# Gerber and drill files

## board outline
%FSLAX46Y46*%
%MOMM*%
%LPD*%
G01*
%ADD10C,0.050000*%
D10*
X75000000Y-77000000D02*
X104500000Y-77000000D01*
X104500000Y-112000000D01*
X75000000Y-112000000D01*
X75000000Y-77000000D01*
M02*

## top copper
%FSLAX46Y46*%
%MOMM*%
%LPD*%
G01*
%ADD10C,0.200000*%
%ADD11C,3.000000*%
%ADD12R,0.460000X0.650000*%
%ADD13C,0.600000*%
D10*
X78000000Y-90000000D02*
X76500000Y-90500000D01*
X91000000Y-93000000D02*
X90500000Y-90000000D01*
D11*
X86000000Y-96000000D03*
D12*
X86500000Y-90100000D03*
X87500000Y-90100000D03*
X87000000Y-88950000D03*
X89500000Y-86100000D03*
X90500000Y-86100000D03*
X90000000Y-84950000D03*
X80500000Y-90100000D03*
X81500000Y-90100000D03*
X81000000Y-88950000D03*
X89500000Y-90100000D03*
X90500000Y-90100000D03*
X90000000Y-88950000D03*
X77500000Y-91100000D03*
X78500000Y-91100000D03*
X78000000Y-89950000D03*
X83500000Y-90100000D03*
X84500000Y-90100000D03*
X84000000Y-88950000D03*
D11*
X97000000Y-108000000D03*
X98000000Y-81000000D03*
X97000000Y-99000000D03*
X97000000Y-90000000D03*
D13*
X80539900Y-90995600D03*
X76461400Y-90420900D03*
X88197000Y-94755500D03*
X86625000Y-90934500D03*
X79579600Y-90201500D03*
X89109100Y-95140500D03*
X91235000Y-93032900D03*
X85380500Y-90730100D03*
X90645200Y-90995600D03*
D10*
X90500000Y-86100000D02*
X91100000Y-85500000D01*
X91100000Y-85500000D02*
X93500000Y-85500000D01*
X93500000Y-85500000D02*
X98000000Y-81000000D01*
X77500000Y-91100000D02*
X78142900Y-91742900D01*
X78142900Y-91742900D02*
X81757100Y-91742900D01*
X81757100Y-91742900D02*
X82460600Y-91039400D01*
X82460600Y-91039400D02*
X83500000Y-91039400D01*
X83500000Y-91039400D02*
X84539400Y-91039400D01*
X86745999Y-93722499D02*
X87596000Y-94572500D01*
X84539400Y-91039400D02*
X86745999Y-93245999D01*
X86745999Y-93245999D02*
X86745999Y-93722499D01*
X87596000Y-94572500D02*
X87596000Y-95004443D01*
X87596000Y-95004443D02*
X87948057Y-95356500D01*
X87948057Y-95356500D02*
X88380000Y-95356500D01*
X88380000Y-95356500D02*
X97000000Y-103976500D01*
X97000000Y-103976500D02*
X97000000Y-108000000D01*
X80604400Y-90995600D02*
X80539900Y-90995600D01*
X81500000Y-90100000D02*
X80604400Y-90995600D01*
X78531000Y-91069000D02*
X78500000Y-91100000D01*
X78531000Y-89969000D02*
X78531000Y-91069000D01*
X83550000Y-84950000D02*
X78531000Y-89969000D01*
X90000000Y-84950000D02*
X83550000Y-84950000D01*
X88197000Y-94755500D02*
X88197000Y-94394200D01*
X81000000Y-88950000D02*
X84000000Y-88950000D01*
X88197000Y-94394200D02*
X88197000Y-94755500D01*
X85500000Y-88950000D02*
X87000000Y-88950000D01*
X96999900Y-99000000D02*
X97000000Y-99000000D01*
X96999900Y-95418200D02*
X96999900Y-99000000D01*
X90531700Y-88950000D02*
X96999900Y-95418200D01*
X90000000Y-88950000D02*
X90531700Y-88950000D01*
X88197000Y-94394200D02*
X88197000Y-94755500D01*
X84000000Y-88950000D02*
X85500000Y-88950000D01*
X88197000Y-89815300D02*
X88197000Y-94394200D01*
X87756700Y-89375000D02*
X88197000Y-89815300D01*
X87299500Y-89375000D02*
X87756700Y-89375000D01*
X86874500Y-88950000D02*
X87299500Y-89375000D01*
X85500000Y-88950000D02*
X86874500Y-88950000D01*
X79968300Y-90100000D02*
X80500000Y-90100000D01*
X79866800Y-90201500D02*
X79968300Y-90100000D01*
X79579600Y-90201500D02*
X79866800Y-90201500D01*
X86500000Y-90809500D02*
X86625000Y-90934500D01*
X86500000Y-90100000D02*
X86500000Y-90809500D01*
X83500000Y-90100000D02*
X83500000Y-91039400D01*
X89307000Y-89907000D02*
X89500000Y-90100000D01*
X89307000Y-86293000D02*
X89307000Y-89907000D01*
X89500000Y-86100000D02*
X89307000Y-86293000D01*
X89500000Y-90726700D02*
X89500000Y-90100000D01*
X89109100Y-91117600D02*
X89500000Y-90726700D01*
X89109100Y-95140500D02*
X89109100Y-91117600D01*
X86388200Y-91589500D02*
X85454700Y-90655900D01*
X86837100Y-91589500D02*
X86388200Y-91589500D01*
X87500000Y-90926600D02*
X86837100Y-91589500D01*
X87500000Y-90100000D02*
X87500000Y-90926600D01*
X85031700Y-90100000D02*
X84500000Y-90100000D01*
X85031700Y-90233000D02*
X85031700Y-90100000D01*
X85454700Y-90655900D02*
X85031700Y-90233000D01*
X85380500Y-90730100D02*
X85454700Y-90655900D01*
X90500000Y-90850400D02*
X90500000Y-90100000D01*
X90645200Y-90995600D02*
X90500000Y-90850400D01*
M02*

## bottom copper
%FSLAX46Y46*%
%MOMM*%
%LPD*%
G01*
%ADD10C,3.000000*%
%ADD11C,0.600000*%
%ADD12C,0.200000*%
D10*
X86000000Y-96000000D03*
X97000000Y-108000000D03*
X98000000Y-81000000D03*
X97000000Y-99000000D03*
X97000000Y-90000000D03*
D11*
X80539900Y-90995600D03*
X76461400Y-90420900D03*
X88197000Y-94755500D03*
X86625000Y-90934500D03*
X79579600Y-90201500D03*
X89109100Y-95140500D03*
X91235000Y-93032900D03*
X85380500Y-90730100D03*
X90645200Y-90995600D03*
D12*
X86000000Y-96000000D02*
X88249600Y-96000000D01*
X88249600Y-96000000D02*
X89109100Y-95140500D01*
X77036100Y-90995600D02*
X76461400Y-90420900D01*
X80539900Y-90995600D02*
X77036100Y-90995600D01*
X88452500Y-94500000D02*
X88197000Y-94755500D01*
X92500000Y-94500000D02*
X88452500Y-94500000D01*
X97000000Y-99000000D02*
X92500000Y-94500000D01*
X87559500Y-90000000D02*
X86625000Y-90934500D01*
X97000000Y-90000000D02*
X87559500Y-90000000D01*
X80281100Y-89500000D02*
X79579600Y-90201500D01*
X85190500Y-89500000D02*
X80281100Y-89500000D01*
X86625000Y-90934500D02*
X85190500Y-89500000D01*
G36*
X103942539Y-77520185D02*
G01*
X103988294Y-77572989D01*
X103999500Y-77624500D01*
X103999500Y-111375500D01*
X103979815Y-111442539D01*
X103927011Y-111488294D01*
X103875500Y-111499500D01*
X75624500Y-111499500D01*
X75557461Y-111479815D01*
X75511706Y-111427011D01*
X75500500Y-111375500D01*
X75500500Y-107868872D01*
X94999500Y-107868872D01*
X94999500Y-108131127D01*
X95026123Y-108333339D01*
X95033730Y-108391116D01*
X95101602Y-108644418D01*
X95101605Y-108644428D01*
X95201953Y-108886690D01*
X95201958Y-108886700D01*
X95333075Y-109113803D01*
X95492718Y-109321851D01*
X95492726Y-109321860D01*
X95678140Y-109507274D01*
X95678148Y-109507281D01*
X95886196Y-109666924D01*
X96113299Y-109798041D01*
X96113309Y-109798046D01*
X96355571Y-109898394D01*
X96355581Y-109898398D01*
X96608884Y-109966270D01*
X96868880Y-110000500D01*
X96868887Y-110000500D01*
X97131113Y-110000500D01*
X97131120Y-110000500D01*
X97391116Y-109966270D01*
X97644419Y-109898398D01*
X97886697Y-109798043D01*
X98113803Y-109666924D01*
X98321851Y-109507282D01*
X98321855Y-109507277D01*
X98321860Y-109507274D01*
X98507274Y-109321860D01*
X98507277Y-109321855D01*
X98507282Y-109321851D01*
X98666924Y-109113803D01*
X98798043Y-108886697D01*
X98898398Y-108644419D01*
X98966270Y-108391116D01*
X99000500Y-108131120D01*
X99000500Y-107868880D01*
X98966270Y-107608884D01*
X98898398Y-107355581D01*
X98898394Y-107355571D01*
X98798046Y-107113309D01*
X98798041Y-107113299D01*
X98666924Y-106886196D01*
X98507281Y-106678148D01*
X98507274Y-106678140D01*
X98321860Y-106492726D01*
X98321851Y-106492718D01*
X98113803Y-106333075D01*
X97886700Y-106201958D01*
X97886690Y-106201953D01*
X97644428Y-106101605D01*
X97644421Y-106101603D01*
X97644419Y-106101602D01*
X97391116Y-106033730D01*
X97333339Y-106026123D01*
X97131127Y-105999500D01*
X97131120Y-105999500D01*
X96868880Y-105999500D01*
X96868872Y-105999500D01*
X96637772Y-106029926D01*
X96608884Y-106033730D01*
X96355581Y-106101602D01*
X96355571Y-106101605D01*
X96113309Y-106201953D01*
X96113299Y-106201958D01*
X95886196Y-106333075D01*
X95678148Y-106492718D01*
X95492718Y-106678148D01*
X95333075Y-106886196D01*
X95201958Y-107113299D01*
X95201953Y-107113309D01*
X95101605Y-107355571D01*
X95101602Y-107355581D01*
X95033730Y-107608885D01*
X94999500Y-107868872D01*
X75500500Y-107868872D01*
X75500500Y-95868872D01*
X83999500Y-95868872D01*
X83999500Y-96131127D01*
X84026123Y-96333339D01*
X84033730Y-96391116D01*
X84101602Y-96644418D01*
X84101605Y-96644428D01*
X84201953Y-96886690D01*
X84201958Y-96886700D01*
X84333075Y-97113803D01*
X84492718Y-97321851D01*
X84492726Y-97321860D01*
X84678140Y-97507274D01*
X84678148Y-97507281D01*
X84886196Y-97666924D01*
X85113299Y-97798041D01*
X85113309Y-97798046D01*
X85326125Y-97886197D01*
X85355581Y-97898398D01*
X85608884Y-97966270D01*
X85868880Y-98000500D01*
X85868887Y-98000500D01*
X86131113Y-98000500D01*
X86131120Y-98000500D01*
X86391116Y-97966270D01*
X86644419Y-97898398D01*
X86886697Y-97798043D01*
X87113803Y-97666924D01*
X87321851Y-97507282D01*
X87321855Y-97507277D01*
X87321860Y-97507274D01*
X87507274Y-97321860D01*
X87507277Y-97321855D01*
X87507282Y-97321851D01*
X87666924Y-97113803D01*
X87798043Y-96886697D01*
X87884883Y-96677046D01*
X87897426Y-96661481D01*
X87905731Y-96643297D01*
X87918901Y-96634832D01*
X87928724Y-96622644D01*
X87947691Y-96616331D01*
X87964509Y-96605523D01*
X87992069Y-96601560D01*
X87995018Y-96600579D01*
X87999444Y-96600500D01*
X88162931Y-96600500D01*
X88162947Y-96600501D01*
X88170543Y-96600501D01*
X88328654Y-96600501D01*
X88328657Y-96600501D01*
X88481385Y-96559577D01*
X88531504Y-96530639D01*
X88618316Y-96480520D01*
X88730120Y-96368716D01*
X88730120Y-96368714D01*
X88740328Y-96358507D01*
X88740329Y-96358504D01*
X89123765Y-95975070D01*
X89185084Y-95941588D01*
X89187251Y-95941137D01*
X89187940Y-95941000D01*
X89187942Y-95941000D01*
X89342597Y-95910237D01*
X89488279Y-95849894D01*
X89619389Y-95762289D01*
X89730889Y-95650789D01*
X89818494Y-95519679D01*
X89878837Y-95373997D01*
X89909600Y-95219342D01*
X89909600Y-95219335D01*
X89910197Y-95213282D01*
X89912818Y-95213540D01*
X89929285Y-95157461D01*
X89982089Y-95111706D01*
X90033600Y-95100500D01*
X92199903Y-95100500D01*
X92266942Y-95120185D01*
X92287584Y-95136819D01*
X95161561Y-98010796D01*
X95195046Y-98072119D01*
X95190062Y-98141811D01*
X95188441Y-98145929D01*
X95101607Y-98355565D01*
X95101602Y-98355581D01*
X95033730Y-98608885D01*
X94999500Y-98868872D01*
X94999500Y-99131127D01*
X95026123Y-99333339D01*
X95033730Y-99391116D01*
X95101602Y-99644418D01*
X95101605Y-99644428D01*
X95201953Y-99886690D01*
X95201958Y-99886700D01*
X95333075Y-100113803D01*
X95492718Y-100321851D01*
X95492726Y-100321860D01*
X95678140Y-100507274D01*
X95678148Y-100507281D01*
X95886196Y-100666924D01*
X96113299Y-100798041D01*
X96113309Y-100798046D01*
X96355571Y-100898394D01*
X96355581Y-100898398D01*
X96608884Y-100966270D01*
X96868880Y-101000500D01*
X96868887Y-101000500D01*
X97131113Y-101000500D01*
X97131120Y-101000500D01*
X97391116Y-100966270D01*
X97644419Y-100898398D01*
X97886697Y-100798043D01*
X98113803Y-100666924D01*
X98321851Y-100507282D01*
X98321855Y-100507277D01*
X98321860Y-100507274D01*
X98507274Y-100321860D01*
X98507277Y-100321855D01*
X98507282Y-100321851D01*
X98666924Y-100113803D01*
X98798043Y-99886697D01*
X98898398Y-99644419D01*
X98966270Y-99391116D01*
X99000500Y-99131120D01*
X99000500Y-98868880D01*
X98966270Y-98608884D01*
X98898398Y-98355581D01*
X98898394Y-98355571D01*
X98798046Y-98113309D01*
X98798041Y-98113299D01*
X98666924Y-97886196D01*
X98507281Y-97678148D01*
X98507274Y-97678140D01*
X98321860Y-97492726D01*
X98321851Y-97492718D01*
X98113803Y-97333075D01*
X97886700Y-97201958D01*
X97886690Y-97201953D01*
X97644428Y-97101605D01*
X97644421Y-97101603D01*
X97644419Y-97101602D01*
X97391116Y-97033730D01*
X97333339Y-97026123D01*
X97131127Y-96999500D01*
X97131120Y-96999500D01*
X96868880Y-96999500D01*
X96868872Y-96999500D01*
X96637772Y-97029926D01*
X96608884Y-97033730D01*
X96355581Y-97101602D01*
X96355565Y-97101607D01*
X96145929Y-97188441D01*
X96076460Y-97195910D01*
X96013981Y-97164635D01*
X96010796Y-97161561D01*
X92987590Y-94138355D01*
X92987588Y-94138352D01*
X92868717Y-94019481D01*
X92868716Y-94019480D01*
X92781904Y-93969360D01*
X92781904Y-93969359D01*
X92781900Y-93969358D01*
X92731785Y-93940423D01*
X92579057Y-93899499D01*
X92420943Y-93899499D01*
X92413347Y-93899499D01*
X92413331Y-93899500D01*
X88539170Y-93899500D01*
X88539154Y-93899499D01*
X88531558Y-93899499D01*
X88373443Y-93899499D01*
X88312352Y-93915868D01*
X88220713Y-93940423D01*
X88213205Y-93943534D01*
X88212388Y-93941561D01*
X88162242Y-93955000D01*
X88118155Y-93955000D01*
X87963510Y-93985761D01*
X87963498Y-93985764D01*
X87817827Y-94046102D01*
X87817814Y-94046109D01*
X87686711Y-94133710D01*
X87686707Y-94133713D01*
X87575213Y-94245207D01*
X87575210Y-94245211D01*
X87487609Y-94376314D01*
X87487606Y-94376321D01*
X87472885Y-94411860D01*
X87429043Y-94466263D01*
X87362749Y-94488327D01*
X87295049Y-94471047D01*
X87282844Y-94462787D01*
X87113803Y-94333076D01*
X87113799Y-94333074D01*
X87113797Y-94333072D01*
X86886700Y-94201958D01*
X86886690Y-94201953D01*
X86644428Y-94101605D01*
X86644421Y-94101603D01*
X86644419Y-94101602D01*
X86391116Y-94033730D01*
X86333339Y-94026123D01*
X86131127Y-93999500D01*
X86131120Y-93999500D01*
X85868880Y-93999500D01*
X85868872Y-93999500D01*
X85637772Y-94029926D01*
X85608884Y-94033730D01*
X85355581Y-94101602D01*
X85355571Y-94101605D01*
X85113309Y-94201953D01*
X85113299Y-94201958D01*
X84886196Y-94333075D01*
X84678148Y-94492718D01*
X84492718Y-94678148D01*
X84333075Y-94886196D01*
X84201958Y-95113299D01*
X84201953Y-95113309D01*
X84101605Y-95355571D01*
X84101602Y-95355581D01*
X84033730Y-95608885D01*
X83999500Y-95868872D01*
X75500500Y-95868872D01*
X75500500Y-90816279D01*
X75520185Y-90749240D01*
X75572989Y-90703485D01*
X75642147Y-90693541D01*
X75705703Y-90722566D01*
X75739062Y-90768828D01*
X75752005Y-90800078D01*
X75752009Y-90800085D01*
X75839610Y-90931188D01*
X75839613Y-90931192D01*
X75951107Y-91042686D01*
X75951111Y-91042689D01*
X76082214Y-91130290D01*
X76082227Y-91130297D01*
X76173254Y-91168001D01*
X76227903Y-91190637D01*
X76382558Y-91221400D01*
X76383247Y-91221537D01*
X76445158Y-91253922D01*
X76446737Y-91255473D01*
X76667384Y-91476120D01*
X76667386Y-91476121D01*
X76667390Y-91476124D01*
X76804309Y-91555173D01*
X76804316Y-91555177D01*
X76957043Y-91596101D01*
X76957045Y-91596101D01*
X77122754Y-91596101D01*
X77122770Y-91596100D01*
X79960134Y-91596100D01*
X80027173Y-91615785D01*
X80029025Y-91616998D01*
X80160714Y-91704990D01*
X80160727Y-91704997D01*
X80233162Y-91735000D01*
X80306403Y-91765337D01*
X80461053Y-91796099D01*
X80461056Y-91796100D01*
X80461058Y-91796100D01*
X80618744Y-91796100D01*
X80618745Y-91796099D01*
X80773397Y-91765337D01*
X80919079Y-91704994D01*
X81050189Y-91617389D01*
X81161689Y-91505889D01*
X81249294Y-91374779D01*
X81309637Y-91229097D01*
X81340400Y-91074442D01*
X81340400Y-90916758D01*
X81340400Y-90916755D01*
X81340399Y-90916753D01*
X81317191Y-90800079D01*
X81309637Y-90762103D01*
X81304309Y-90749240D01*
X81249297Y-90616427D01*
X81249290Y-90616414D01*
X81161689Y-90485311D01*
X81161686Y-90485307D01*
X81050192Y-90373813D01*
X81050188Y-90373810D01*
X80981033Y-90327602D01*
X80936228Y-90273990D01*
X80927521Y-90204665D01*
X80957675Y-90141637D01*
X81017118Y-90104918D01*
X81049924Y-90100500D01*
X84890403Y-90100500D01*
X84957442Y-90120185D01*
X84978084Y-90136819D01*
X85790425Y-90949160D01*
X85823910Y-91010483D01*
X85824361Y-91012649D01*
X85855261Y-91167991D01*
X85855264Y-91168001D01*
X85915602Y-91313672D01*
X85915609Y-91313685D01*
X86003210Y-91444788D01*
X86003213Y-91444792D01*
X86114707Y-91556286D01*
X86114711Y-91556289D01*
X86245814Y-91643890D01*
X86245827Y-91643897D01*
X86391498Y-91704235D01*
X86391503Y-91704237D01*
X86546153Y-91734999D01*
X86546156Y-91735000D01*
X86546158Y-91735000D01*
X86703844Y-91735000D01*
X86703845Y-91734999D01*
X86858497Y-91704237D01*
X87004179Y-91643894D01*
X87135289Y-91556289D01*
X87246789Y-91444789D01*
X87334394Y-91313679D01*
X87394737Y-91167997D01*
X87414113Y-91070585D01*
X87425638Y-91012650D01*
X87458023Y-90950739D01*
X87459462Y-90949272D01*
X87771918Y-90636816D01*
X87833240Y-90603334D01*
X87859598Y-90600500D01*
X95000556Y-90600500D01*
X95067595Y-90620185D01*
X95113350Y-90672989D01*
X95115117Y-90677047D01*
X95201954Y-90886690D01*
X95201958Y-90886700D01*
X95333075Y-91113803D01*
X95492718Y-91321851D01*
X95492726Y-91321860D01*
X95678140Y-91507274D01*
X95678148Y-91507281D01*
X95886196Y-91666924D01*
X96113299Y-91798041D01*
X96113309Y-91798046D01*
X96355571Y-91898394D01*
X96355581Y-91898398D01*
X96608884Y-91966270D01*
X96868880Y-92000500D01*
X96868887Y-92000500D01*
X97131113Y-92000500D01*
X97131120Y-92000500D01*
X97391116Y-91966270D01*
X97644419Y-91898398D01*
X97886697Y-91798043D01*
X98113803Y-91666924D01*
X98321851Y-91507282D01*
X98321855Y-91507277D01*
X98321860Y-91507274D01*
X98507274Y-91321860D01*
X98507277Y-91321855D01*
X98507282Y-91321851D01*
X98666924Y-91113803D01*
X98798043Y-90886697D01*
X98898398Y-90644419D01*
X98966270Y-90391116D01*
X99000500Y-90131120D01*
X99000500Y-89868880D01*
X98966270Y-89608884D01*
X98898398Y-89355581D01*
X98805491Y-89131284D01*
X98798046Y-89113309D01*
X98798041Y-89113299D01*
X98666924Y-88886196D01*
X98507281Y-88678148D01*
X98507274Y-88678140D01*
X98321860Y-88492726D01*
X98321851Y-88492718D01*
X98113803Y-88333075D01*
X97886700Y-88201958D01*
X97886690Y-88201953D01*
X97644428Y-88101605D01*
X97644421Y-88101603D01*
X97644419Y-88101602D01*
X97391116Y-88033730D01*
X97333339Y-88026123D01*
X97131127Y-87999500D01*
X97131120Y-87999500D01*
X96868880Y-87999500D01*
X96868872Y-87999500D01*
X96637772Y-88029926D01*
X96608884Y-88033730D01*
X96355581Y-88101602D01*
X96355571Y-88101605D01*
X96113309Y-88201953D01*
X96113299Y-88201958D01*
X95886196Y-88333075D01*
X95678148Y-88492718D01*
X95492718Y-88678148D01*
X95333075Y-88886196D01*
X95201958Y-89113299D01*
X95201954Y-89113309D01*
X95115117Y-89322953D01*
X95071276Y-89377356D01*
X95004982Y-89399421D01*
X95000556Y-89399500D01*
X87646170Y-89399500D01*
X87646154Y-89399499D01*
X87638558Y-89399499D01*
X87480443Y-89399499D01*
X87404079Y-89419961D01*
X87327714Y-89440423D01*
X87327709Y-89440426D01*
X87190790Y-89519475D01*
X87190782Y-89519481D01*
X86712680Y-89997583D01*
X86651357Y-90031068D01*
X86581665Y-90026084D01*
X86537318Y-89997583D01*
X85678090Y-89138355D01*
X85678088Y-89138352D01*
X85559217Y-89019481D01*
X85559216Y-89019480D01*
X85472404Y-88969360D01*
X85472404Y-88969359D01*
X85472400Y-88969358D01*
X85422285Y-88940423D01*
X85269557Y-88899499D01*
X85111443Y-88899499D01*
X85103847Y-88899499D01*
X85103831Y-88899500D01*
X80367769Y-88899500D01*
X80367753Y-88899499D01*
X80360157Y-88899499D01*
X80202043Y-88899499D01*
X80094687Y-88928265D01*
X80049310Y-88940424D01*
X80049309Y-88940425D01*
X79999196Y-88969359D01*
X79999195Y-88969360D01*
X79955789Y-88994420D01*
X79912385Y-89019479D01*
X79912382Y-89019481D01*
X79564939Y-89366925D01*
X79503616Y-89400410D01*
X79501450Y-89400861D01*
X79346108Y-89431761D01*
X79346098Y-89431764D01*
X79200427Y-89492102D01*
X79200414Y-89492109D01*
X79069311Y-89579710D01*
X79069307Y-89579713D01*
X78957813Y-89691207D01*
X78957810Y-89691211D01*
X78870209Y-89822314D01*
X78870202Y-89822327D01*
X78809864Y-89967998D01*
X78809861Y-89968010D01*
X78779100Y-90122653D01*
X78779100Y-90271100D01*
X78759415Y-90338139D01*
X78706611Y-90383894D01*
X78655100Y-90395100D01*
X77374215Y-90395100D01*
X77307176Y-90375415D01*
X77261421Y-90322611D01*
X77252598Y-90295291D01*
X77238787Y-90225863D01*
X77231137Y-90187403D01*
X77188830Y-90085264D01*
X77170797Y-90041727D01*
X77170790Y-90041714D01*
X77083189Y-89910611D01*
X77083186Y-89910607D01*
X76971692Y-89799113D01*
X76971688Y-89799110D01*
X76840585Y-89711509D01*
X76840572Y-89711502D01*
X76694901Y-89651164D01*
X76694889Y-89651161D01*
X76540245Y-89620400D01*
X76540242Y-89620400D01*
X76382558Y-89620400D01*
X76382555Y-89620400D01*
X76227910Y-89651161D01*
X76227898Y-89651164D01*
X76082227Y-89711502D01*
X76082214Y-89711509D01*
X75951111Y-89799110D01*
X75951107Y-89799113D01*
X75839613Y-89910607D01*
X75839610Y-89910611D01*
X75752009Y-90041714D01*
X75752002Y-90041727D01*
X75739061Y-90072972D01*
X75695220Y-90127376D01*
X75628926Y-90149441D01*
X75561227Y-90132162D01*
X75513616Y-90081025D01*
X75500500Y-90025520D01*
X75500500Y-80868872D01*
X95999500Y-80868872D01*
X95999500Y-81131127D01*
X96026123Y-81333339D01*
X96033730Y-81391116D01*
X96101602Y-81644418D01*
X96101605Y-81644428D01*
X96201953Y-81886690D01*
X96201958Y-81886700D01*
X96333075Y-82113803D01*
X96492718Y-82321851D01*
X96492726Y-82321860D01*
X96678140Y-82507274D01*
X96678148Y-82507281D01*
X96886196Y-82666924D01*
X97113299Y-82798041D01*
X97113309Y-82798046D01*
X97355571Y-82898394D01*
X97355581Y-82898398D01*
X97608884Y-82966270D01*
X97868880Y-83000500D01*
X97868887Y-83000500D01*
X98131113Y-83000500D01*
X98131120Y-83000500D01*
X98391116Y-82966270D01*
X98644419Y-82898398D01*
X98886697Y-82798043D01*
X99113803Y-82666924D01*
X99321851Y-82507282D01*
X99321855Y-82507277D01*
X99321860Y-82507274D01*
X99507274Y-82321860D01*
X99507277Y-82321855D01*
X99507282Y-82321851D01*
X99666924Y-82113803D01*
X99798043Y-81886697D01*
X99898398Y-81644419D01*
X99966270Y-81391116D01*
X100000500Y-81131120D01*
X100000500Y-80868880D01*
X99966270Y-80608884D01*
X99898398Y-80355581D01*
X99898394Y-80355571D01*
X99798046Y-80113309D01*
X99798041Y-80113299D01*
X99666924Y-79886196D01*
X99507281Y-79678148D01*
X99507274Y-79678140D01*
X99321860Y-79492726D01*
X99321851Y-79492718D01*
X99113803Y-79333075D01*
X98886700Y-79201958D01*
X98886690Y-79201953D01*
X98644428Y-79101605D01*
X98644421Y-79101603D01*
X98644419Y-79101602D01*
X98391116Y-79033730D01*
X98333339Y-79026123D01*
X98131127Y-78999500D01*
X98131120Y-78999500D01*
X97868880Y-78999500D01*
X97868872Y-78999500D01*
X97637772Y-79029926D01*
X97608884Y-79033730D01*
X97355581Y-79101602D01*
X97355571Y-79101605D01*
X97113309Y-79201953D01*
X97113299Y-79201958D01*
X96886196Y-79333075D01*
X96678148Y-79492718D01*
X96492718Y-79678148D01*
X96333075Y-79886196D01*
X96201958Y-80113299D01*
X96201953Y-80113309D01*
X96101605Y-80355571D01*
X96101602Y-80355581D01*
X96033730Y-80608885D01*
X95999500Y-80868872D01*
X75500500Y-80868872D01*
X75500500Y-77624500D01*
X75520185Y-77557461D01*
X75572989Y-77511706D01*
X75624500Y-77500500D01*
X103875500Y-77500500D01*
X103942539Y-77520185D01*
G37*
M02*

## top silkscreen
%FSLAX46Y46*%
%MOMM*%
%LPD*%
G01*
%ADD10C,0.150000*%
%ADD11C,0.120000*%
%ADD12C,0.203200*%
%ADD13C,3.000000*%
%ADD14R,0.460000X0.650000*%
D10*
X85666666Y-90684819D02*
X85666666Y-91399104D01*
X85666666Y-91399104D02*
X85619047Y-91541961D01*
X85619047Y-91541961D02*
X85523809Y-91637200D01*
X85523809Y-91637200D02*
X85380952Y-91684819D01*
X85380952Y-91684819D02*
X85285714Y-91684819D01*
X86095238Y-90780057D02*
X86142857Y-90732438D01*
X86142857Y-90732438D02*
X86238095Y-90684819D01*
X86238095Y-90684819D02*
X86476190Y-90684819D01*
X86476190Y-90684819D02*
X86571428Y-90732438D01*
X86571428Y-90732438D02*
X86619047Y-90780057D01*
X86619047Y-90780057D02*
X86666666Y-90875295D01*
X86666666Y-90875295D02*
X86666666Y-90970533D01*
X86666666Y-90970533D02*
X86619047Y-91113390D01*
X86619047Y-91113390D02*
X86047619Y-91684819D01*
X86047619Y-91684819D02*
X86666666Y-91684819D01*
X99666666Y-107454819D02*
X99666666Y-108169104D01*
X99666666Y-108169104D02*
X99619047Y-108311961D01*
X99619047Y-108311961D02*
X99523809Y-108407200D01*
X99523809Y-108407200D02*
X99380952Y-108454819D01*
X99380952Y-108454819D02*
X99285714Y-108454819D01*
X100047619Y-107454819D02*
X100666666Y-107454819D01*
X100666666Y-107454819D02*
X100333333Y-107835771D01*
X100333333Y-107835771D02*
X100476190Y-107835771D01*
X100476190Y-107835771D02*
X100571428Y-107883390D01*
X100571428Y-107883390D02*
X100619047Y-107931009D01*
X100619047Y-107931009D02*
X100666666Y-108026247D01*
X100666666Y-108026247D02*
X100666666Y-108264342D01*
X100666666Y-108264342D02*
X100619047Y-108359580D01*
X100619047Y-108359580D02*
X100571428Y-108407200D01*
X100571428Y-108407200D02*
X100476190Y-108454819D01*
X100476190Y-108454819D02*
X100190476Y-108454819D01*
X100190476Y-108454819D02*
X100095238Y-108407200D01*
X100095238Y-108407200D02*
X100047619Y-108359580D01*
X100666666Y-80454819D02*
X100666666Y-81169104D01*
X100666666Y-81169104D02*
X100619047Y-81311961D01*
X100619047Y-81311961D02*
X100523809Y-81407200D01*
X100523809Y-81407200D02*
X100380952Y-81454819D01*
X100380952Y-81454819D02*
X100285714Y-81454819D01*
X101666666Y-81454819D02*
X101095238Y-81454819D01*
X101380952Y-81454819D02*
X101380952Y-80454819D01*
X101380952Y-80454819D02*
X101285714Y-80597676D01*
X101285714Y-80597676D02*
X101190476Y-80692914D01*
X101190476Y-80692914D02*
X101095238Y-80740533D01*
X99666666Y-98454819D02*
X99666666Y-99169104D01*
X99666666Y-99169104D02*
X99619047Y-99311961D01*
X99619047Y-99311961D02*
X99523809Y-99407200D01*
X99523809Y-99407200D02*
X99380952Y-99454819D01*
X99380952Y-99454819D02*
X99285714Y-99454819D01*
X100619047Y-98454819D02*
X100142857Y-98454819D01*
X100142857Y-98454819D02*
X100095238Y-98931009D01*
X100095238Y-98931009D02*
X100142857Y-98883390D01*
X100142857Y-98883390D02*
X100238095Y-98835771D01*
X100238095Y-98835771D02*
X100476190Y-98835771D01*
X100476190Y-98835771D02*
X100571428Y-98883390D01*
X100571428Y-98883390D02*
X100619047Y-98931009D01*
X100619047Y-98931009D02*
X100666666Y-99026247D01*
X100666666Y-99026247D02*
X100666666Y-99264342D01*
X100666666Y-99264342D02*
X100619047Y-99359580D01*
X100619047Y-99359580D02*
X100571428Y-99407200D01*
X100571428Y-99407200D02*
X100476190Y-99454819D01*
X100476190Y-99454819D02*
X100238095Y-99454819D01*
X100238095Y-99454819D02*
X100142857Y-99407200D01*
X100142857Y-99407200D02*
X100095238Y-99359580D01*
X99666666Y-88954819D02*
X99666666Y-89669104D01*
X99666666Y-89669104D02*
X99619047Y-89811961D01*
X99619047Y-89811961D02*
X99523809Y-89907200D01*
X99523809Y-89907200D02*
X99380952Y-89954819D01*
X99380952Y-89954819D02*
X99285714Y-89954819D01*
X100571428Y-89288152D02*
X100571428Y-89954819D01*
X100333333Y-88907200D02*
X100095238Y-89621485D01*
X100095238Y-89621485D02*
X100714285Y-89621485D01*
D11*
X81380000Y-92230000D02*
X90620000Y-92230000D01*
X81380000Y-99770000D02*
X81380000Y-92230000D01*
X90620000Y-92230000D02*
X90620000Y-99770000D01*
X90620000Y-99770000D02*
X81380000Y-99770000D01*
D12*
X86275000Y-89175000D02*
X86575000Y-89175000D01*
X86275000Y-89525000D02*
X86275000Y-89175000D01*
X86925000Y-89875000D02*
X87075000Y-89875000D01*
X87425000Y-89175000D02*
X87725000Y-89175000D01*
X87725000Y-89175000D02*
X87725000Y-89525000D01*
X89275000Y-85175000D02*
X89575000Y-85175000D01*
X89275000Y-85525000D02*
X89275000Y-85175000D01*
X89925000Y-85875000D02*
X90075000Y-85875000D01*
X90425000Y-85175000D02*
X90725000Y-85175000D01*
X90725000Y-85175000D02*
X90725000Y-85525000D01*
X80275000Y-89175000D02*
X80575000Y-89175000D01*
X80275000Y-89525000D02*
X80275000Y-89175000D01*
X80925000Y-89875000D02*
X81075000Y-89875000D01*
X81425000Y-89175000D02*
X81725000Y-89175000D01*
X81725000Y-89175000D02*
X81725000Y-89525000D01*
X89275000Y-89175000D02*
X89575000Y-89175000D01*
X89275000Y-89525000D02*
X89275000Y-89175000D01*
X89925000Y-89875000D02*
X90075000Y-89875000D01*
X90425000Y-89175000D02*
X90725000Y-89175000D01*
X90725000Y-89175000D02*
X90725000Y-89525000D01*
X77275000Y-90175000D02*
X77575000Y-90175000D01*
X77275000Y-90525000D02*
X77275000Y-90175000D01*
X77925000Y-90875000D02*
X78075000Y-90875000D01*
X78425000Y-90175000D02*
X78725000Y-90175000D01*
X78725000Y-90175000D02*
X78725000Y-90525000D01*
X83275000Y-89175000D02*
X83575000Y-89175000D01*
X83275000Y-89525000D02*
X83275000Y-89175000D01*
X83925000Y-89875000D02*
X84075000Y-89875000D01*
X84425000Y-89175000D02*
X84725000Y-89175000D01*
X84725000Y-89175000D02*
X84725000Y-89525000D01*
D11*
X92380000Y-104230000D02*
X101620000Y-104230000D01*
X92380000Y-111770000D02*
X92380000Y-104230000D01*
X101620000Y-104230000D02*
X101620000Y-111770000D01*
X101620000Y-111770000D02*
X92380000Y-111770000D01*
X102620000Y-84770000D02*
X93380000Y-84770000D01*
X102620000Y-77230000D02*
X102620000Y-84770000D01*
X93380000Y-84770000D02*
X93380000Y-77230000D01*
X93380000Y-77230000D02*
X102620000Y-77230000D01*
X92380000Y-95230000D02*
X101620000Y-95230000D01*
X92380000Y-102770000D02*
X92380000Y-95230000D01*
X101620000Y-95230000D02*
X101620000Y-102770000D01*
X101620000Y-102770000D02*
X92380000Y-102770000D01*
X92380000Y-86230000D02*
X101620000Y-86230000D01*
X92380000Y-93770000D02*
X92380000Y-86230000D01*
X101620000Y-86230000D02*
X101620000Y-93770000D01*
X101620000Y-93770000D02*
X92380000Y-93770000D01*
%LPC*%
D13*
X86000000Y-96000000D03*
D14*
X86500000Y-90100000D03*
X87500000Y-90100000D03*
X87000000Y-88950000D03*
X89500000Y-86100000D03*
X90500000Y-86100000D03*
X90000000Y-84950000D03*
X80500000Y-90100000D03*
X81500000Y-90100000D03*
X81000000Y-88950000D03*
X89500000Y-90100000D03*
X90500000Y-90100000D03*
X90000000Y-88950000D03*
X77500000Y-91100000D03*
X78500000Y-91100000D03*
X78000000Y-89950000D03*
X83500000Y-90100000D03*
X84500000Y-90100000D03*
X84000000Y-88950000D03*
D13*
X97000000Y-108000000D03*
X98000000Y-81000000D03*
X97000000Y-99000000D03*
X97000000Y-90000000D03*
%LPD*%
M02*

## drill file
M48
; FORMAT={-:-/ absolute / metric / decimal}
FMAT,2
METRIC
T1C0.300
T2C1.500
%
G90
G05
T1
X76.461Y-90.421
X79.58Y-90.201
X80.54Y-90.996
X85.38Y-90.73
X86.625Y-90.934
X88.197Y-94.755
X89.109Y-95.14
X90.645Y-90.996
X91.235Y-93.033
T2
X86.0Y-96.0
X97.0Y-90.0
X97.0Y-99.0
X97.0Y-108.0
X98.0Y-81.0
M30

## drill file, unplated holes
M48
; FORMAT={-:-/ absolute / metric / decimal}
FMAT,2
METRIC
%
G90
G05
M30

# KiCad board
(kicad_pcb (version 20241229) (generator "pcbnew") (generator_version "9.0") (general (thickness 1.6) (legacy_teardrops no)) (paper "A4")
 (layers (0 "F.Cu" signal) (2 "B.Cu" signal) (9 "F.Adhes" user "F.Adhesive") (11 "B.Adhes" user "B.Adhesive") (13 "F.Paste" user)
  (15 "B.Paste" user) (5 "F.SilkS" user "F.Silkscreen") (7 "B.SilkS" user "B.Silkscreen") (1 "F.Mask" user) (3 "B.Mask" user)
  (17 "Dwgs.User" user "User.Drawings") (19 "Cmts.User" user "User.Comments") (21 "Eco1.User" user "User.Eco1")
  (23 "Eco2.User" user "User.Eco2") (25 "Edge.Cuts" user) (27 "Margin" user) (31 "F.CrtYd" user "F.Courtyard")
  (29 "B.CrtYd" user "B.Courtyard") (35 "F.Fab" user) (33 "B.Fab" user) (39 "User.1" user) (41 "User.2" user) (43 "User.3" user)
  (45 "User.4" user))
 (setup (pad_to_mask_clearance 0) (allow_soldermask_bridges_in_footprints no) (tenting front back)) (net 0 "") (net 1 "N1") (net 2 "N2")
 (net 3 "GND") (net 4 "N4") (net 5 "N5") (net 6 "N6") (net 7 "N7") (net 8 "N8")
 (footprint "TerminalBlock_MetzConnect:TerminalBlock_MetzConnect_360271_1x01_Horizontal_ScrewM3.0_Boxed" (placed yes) (layer "F.Cu")
  (at 86 96)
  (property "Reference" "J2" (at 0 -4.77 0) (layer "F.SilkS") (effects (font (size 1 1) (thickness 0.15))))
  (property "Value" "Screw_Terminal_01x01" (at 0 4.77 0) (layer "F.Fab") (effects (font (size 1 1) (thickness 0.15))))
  (fp_line (start -4.62 -3.77) (end 4.62 -3.77) (stroke (width 0.12) (type solid)) (layer "F.SilkS"))
  (fp_line (start -4.62 3.77) (end -4.62 -3.77) (stroke (width 0.12) (type solid)) (layer "F.SilkS"))
  (fp_line (start 4.62 -3.77) (end 4.62 3.77) (stroke (width 0.12) (type solid)) (layer "F.SilkS"))
  (fp_line (start 4.62 3.77) (end -4.62 3.77) (stroke (width 0.12) (type solid)) (layer "F.SilkS"))
  (pad "1" thru_hole circle (at 0 0) (size 3 3) (drill 1.5) (layers "*.Cu" "*.Mask") (remove_unused_layers no) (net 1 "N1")))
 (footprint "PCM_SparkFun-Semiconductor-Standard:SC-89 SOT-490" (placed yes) (layer "F.Cu") (at 87 89)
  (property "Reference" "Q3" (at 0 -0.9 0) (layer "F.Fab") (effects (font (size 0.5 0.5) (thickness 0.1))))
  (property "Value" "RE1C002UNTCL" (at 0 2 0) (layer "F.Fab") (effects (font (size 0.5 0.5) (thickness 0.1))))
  (fp_line (start -0.725 0.175) (end -0.425 0.175) (stroke (width 0.2032) (type solid)) (layer "F.SilkS"))
  (fp_line (start -0.725 0.525) (end -0.725 0.175) (stroke (width 0.2032) (type solid)) (layer "F.SilkS"))
  (fp_line (start -0.075 0.875) (end 0.075 0.875) (stroke (width 0.2032) (type solid)) (layer "F.SilkS"))
  (fp_line (start 0.425 0.175) (end 0.725 0.175) (stroke (width 0.2032) (type solid)) (layer "F.SilkS"))
  (fp_line (start 0.725 0.175) (end 0.725 0.525) (stroke (width 0.2032) (type solid)) (layer "F.SilkS"))
  (pad "1" smd rect (at -0.5 1.1) (size 0.46 0.65) (layers "F.Cu" "F.Mask" "F.Paste") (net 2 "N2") (thermal_bridge_angle 0))
  (pad "2" smd rect (at 0.5 1.1) (size 0.46 0.65) (layers "F.Cu" "F.Mask" "F.Paste") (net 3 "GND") (thermal_bridge_angle 0))
  (pad "3" smd rect (at 0 -0.05) (size 0.46 0.65) (layers "F.Cu" "F.Mask" "F.Paste") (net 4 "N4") (thermal_bridge_angle 0)))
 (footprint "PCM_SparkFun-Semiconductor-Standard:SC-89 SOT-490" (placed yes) (layer "F.Cu") (at 90 85)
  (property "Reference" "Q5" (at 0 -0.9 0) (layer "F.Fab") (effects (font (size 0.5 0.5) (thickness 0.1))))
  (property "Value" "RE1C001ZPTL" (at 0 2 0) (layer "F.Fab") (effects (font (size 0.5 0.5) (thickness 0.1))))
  (fp_line (start -0.725 0.175) (end -0.425 0.175) (stroke (width 0.2032) (type solid)) (layer "F.SilkS"))
  (fp_line (start -0.725 0.525) (end -0.725 0.175) (stroke (width 0.2032) (type solid)) (layer "F.SilkS"))
  (fp_line (start -0.075 0.875) (end 0.075 0.875) (stroke (width 0.2032) (type solid)) (layer "F.SilkS"))
  (fp_line (start 0.425 0.175) (end 0.725 0.175) (stroke (width 0.2032) (type solid)) (layer "F.SilkS"))
  (fp_line (start 0.725 0.175) (end 0.725 0.525) (stroke (width 0.2032) (type solid)) (layer "F.SilkS"))
  (pad "1" smd rect (at -0.5 1.1) (size 0.46 0.65) (layers "F.Cu" "F.Mask" "F.Paste") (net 1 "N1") (thermal_bridge_angle 0))
  (pad "2" smd rect (at 0.5 1.1) (size 0.46 0.65) (layers "F.Cu" "F.Mask" "F.Paste") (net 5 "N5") (thermal_bridge_angle 0))
  (pad "3" smd rect (at 0 -0.05) (size 0.46 0.65) (layers "F.Cu" "F.Mask" "F.Paste") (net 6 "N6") (thermal_bridge_angle 0)))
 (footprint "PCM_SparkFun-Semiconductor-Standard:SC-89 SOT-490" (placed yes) (layer "F.Cu") (at 81 89)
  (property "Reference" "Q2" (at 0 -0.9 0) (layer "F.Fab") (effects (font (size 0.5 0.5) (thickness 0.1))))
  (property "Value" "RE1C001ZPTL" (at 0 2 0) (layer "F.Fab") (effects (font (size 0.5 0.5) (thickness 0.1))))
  (fp_line (start -0.725 0.175) (end -0.425 0.175) (stroke (width 0.2032) (type solid)) (layer "F.SilkS"))
  (fp_line (start -0.725 0.525) (end -0.725 0.175) (stroke (width 0.2032) (type solid)) (layer "F.SilkS"))
  (fp_line (start -0.075 0.875) (end 0.075 0.875) (stroke (width 0.2032) (type solid)) (layer "F.SilkS"))
  (fp_line (start 0.425 0.175) (end 0.725 0.175) (stroke (width 0.2032) (type solid)) (layer "F.SilkS"))
  (fp_line (start 0.725 0.175) (end 0.725 0.525) (stroke (width 0.2032) (type solid)) (layer "F.SilkS"))
  (pad "1" smd rect (at -0.5 1.1) (size 0.46 0.65) (layers "F.Cu" "F.Mask" "F.Paste") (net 2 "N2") (thermal_bridge_angle 0))
  (pad "2" smd rect (at 0.5 1.1) (size 0.46 0.65) (layers "F.Cu" "F.Mask" "F.Paste") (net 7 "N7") (thermal_bridge_angle 0))
  (pad "3" smd rect (at 0 -0.05) (size 0.46 0.65) (layers "F.Cu" "F.Mask" "F.Paste") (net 4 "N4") (thermal_bridge_angle 0)))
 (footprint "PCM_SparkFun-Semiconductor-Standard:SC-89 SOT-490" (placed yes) (layer "F.Cu") (at 90 89)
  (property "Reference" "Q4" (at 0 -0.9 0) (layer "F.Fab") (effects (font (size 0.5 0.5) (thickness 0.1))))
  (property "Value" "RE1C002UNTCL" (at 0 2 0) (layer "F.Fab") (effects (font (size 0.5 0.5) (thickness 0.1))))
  (fp_line (start -0.725 0.175) (end -0.425 0.175) (stroke (width 0.2032) (type solid)) (layer "F.SilkS"))
  (fp_line (start -0.725 0.525) (end -0.725 0.175) (stroke (width 0.2032) (type solid)) (layer "F.SilkS"))
  (fp_line (start -0.075 0.875) (end 0.075 0.875) (stroke (width 0.2032) (type solid)) (layer "F.SilkS"))
  (fp_line (start 0.425 0.175) (end 0.725 0.175) (stroke (width 0.2032) (type solid)) (layer "F.SilkS"))
  (fp_line (start 0.725 0.175) (end 0.725 0.525) (stroke (width 0.2032) (type solid)) (layer "F.SilkS"))
  (pad "1" smd rect (at -0.5 1.1) (size 0.46 0.65) (layers "F.Cu" "F.Mask" "F.Paste") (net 1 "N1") (thermal_bridge_angle 0))
  (pad "2" smd rect (at 0.5 1.1) (size 0.46 0.65) (layers "F.Cu" "F.Mask" "F.Paste") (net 3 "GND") (thermal_bridge_angle 0))
  (pad "3" smd rect (at 0 -0.05) (size 0.46 0.65) (layers "F.Cu" "F.Mask" "F.Paste") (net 4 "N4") (thermal_bridge_angle 0)))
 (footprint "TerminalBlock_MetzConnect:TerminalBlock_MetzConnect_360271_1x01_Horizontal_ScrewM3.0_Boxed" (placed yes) (layer "F.Cu")
  (at 97 90)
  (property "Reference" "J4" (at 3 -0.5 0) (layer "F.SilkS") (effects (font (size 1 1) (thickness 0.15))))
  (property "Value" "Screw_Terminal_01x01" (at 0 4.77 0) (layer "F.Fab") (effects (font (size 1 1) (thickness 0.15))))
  (fp_line (start -4.62 -3.77) (end 4.62 -3.77) (stroke (width 0.12) (type solid)) (layer "F.SilkS"))
  (fp_line (start -4.62 3.77) (end -4.62 -3.77) (stroke (width 0.12) (type solid)) (layer "F.SilkS"))
  (fp_line (start 4.62 -3.77) (end 4.62 3.77) (stroke (width 0.12) (type solid)) (layer "F.SilkS"))
  (fp_line (start 4.62 3.77) (end -4.62 3.77) (stroke (width 0.12) (type solid)) (layer "F.SilkS"))
  (pad "1" thru_hole circle (at 0 0) (size 3 3) (drill 1.5) (layers "*.Cu" "*.Mask") (remove_unused_layers no) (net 2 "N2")))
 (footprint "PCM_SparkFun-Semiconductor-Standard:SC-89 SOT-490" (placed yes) (layer "F.Cu") (at 78 90)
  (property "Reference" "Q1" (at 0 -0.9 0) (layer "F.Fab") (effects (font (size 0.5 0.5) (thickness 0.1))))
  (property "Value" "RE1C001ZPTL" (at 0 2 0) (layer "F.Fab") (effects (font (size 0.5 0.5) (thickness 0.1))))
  (fp_line (start -0.725 0.175) (end -0.425 0.175) (stroke (width 0.2032) (type solid)) (layer "F.SilkS"))
  (fp_line (start -0.725 0.525) (end -0.725 0.175) (stroke (width 0.2032) (type solid)) (layer "F.SilkS"))
  (fp_line (start -0.075 0.875) (end 0.075 0.875) (stroke (width 0.2032) (type solid)) (layer "F.SilkS"))
  (fp_line (start 0.425 0.175) (end 0.725 0.175) (stroke (width 0.2032) (type solid)) (layer "F.SilkS"))
  (fp_line (start 0.725 0.175) (end 0.725 0.525) (stroke (width 0.2032) (type solid)) (layer "F.SilkS"))
  (pad "1" smd rect (at -0.5 1.1) (size 0.46 0.65) (layers "F.Cu" "F.Mask" "F.Paste") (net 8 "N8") (thermal_bridge_angle 0))
  (pad "2" smd rect (at 0.5 1.1) (size 0.46 0.65) (layers "F.Cu" "F.Mask" "F.Paste") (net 6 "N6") (thermal_bridge_angle 0))
  (pad "3" smd rect (at 0 -0.05) (size 0.46 0.65) (layers "F.Cu" "F.Mask" "F.Paste") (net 7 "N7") (thermal_bridge_angle 0)))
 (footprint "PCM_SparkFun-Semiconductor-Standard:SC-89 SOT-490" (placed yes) (layer "F.Cu") (at 84 89)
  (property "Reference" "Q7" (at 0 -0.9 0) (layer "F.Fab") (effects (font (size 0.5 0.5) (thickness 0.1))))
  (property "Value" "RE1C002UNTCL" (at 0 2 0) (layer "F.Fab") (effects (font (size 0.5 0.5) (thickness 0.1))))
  (fp_line (start -0.725 0.175) (end -0.425 0.175) (stroke (width 0.2032) (type solid)) (layer "F.SilkS"))
  (fp_line (start -0.725 0.525) (end -0.725 0.175) (stroke (width 0.2032) (type solid)) (layer "F.SilkS"))
  (fp_line (start -0.075 0.875) (end 0.075 0.875) (stroke (width 0.2032) (type solid)) (layer "F.SilkS"))
  (fp_line (start 0.425 0.175) (end 0.725 0.175) (stroke (width 0.2032) (type solid)) (layer "F.SilkS"))
  (fp_line (start 0.725 0.175) (end 0.725 0.525) (stroke (width 0.2032) (type solid)) (layer "F.SilkS"))
  (pad "1" smd rect (at -0.5 1.1) (size 0.46 0.65) (layers "F.Cu" "F.Mask" "F.Paste") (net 8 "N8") (thermal_bridge_angle 0))
  (pad "2" smd rect (at 0.5 1.1) (size 0.46 0.65) (layers "F.Cu" "F.Mask" "F.Paste") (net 3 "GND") (thermal_bridge_angle 0))
  (pad "3" smd rect (at 0 -0.05) (size 0.46 0.65) (layers "F.Cu" "F.Mask" "F.Paste") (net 4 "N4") (thermal_bridge_angle 0)))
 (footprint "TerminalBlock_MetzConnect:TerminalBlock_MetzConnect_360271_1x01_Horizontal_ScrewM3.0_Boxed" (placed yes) (layer "F.Cu")
  (at 97 108)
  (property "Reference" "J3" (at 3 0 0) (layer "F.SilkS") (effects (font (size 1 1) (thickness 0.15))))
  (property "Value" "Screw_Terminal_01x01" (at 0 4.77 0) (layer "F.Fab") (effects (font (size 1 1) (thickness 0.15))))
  (fp_line (start -4.62 -3.77) (end 4.62 -3.77) (stroke (width 0.12) (type solid)) (layer "F.SilkS"))
  (fp_line (start -4.62 3.77) (end -4.62 -3.77) (stroke (width 0.12) (type solid)) (layer "F.SilkS"))
  (fp_line (start 4.62 -3.77) (end 4.62 3.77) (stroke (width 0.12) (type solid)) (layer "F.SilkS"))
  (fp_line (start 4.62 3.77) (end -4.62 3.77) (stroke (width 0.12) (type solid)) (layer "F.SilkS"))
  (pad "1" thru_hole circle (at 0 0) (size 3 3) (drill 1.5) (layers "*.Cu" "*.Mask") (remove_unused_layers no) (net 8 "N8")))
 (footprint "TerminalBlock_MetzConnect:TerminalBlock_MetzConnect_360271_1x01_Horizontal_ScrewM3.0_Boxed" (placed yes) (layer "F.Cu")
  (at 98 81)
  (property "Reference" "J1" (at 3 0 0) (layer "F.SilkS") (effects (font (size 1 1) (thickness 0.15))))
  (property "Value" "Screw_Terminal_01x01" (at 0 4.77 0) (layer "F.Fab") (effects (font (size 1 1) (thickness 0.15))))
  (fp_line (start -4.62 -3.77) (end 4.62 -3.77) (stroke (width 0.12) (type solid)) (layer "F.SilkS"))
  (fp_line (start -4.62 3.77) (end -4.62 -3.77) (stroke (width 0.12) (type solid)) (layer "F.SilkS"))
  (fp_line (start 4.62 -3.77) (end 4.62 3.77) (stroke (width 0.12) (type solid)) (layer "F.SilkS"))
  (fp_line (start 4.62 3.77) (end -4.62 3.77) (stroke (width 0.12) (type solid)) (layer "F.SilkS"))
  (pad "1" thru_hole circle (at 0 0) (size 3 3) (drill 1.5) (layers "*.Cu" "*.Mask") (remove_unused_layers no) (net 5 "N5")))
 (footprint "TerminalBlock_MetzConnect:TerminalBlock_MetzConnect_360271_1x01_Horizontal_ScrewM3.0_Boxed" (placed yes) (layer "F.Cu")
  (at 97 99)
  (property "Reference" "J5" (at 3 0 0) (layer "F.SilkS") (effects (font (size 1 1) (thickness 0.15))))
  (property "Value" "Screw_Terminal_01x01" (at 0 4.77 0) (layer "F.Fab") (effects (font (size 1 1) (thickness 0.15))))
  (fp_line (start -4.62 -3.77) (end 4.62 -3.77) (stroke (width 0.12) (type solid)) (layer "F.SilkS"))
  (fp_line (start -4.62 3.77) (end -4.62 -3.77) (stroke (width 0.12) (type solid)) (layer "F.SilkS"))
  (fp_line (start 4.62 -3.77) (end 4.62 3.77) (stroke (width 0.12) (type solid)) (layer "F.SilkS"))
  (fp_line (start 4.62 3.77) (end -4.62 3.77) (stroke (width 0.12) (type solid)) (layer "F.SilkS"))
  (pad "1" thru_hole circle (at 0 0) (size 3 3) (drill 1.5) (layers "*.Cu" "*.Mask") (remove_unused_layers no) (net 4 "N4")))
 (gr_line (start 91 93) (end 90.5 90) (stroke (width 0.2) (type default)) (layer "F.Cu") (net 3))
 (gr_line (start 78 90) (end 76.5 90.5) (stroke (width 0.2) (type default)) (layer "F.Cu") (net 7))
 (gr_rect (start 75 77) (end 104.5 112) (stroke (width 0.05) (type default)) (fill no) (layer "Edge.Cuts"))
 (segment (start 90.5 86.1) (end 91.1 85.5) (width 0.2) (layer "F.Cu") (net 5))
 (segment (start 93.5 85.5) (end 98 81) (width 0.2) (layer "F.Cu") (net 5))
 (segment (start 91.1 85.5) (end 93.5 85.5) (width 0.2) (layer "F.Cu") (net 5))
 (segment (start 89.307 86.293) (end 89.307 89.907) (width 0.2) (layer "F.Cu") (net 1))
 (segment (start 89.5 86.1) (end 89.307 86.293) (width 0.2) (layer "F.Cu") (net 1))
 (segment (start 89.307 89.907) (end 89.5 90.1) (width 0.2) (layer "F.Cu") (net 1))
 (segment (start 89.1091 91.1176) (end 89.5 90.7267) (width 0.2) (layer "F.Cu") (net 1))
 (segment (start 89.1091 95.1405) (end 89.1091 91.1176) (width 0.2) (layer "F.Cu") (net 1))
 (segment (start 89.5 90.7267) (end 89.5 90.1) (width 0.2) (layer "F.Cu") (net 1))
 (via (at 89.1091 95.1405) (size 0.6) (drill 0.3) (layers "F.Cu" "B.Cu") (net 1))
 (segment (start 86 96) (end 88.2496 96) (width 0.2) (layer "B.Cu") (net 1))
 (segment (start 88.2496 96) (end 89.1091 95.1405) (width 0.2) (layer "B.Cu") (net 1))
 (segment (start 77.5 91.1) (end 78.1429 91.7429) (width 0.2) (layer "F.Cu") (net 8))
 (segment (start 83.5 91.0394) (end 84.5394 91.0394) (width 0.2) (layer "F.Cu") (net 8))
 (segment (start 88.38 95.3565) (end 97 103.9765) (width 0.2) (layer "F.Cu") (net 8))
 (segment (start 86.745999 93.245999) (end 86.745999 93.722499) (width 0.2) (layer "F.Cu") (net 8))
 (segment (start 87.948057 95.3565) (end 88.38 95.3565) (width 0.2) (layer "F.Cu") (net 8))
 (segment (start 83.5 90.1) (end 83.5 91.0394) (width 0.2) (layer "F.Cu") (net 8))
 (segment (start 87.596 94.5725) (end 87.596 95.004443) (width 0.2) (layer "F.Cu") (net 8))
 (segment (start 81.7571 91.7429) (end 82.4606 91.0394) (width 0.2) (layer "F.Cu") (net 8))
 (segment (start 84.5394 91.0394) (end 86.745999 93.245999) (width 0.2) (layer "F.Cu") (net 8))
 (segment (start 82.4606 91.0394) (end 83.5 91.0394) (width 0.2) (layer "F.Cu") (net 8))
 (segment (start 97 103.9765) (end 97 108) (width 0.2) (layer "F.Cu") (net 8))
 (segment (start 78.1429 91.7429) (end 81.7571 91.7429) (width 0.2) (layer "F.Cu") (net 8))
 (segment (start 86.745999 93.722499) (end 87.596 94.5725) (width 0.2) (layer "F.Cu") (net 8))
 (segment (start 87.596 95.004443) (end 87.948057 95.3565) (width 0.2) (layer "F.Cu") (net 8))
 (segment (start 79.5796 90.2015) (end 79.8668 90.2015) (width 0.2) (layer "F.Cu") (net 2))
 (segment (start 79.9683 90.1) (end 80.5 90.1) (width 0.2) (layer "F.Cu") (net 2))
 (segment (start 86.5 90.8095) (end 86.625 90.9345) (width 0.2) (layer "F.Cu") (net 2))
 (segment (start 79.8668 90.2015) (end 79.9683 90.1) (width 0.2) (layer "F.Cu") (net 2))
 (segment (start 86.5 90.1) (end 86.5 90.8095) (width 0.2) (layer "F.Cu") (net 2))
 (via (at 79.5796 90.2015) (size 0.6) (drill 0.3) (layers "F.Cu" "B.Cu") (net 2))
 (via (at 86.625 90.9345) (size 0.6) (drill 0.3) (layers "F.Cu" "B.Cu") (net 2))
 (segment (start 80.2811 89.5) (end 79.5796 90.2015) (width 0.2) (layer "B.Cu") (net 2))
 (segment (start 87.5595 90) (end 86.625 90.9345) (width 0.2) (layer "B.Cu") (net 2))
 (segment (start 97 90) (end 87.5595 90) (width 0.2) (layer "B.Cu") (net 2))
 (segment (start 86.625 90.9345) (end 85.1905 89.5) (width 0.2) (layer "B.Cu") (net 2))
 (segment (start 85.1905 89.5) (end 80.2811 89.5) (width 0.2) (layer "B.Cu") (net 2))
 (segment (start 90 88.95) (end 90.5317 88.95) (width 0.2) (layer "F.Cu") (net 4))
 (segment (start 96.9999 99) (end 97 99) (width 0.2) (layer "F.Cu") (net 4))
 (segment (start 84 88.95) (end 85.5 88.95) (width 0.2) (layer "F.Cu") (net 4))
 (segment (start 88.197 89.8153) (end 88.197 94.3942) (width 0.2) (layer "F.Cu") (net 4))
 (segment (start 90.5317 88.95) (end 96.9999 95.4182) (width 0.2) (layer "F.Cu") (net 4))
 (segment (start 86.8745 88.95) (end 87.2995 89.375) (width 0.2) (layer "F.Cu") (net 4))
 (segment (start 87.2995 89.375) (end 87.7567 89.375) (width 0.2) (layer "F.Cu") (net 4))
 (segment (start 81 88.95) (end 84 88.95) (width 0.2) (layer "F.Cu") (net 4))
 (segment (start 85.5 88.95) (end 87 88.95) (width 0.2) (layer "F.Cu") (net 4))
 (segment (start 88.197 94.3942) (end 88.197 94.7555) (width 0.2) (layer "F.Cu") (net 4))
 (segment (start 85.5 88.95) (end 86.8745 88.95) (width 0.2) (layer "F.Cu") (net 4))
 (segment (start 87.7567 89.375) (end 88.197 89.8153) (width 0.2) (layer "F.Cu") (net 4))
 (segment (start 88.197 94.3942) (end 88.197 94.7555) (width 0.2) (layer "F.Cu") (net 4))
 (segment (start 88.197 94.7555) (end 88.197 94.3942) (width 0.2) (layer "F.Cu") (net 4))
 (segment (start 96.9999 95.4182) (end 96.9999 99) (width 0.2) (layer "F.Cu") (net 4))
 (via (at 88.197 94.7555) (size 0.6) (drill 0.3) (layers "F.Cu" "B.Cu") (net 4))
 (segment (start 92.5 94.5) (end 88.4525 94.5) (width 0.2) (layer "B.Cu") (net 4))
 (segment (start 88.4525 94.5) (end 88.197 94.7555) (width 0.2) (layer "B.Cu") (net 4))
 (segment (start 97 99) (end 92.5 94.5) (width 0.2) (layer "B.Cu") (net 4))
 (segment (start 78.531 91.069) (end 78.5 91.1) (width 0.2) (layer "F.Cu") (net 6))
 (segment (start 83.55 84.95) (end 78.531 89.969) (width 0.2) (layer "F.Cu") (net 6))
 (segment (start 90 84.95) (end 83.55 84.95) (width 0.2) (layer "F.Cu") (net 6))
 (segment (start 78.531 89.969) (end 78.531 91.069) (width 0.2) (layer "F.Cu") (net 6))
 (segment (start 81.5 90.1) (end 80.6044 90.9956) (width 0.2) (layer "F.Cu") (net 7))
 (segment (start 80.6044 90.9956) (end 80.5399 90.9956) (width 0.2) (layer "F.Cu") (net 7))
 (via (at 76.4614 90.4209) (size 0.6) (drill 0.3) (layers "F.Cu" "B.Cu") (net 7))
 (via (at 80.5399 90.9956) (size 0.6) (drill 0.3) (layers "F.Cu" "B.Cu") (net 7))
 (segment (start 80.5399 90.9956) (end 77.0361 90.9956) (width 0.2) (layer "B.Cu") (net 7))
 (segment (start 77.0361 90.9956) (end 76.4614 90.4209) (width 0.2) (layer "B.Cu") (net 7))
 (segment (start 85.4547 90.6559) (end 85.0317 90.233) (width 0.2) (layer "F.Cu") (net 3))
 (segment (start 85.0317 90.233) (end 85.0317 90.1) (width 0.2) (layer "F.Cu") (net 3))
 (segment (start 90.6452 90.9956) (end 90.5 90.8504) (width 0.2) (layer "F.Cu") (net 3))
 (segment (start 87.5 90.9266) (end 86.8371 91.5895) (width 0.2) (layer "F.Cu") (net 3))
 (segment (start 85.0317 90.1) (end 84.5 90.1) (width 0.2) (layer "F.Cu") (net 3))
 (segment (start 86.3882 91.5895) (end 85.4547 90.6559) (width 0.2) (layer "F.Cu") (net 3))
 (segment (start 86.8371 91.5895) (end 86.3882 91.5895) (width 0.2) (layer "F.Cu") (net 3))
 (segment (start 85.3805 90.7301) (end 85.4547 90.6559) (width 0.2) (layer "F.Cu") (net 3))
 (segment (start 87.5 90.1) (end 87.5 90.9266) (width 0.2) (layer "F.Cu") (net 3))
 (segment (start 90.5 90.8504) (end 90.5 90.1) (width 0.2) (layer "F.Cu") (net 3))
 (via (at 91.235 93.0329) (size 0.6) (drill 0.3) (layers "F.Cu" "B.Cu") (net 3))
 (via (at 85.3805 90.7301) (size 0.6) (drill 0.3) (layers "F.Cu" "B.Cu") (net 3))
 (via (at 90.6452 90.9956) (size 0.6) (drill 0.3) (layers "F.Cu" "B.Cu") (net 3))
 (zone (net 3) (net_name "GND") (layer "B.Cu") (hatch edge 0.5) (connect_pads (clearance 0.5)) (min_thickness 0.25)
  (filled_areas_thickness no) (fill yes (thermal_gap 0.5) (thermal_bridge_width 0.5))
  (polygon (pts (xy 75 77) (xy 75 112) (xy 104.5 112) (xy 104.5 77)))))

